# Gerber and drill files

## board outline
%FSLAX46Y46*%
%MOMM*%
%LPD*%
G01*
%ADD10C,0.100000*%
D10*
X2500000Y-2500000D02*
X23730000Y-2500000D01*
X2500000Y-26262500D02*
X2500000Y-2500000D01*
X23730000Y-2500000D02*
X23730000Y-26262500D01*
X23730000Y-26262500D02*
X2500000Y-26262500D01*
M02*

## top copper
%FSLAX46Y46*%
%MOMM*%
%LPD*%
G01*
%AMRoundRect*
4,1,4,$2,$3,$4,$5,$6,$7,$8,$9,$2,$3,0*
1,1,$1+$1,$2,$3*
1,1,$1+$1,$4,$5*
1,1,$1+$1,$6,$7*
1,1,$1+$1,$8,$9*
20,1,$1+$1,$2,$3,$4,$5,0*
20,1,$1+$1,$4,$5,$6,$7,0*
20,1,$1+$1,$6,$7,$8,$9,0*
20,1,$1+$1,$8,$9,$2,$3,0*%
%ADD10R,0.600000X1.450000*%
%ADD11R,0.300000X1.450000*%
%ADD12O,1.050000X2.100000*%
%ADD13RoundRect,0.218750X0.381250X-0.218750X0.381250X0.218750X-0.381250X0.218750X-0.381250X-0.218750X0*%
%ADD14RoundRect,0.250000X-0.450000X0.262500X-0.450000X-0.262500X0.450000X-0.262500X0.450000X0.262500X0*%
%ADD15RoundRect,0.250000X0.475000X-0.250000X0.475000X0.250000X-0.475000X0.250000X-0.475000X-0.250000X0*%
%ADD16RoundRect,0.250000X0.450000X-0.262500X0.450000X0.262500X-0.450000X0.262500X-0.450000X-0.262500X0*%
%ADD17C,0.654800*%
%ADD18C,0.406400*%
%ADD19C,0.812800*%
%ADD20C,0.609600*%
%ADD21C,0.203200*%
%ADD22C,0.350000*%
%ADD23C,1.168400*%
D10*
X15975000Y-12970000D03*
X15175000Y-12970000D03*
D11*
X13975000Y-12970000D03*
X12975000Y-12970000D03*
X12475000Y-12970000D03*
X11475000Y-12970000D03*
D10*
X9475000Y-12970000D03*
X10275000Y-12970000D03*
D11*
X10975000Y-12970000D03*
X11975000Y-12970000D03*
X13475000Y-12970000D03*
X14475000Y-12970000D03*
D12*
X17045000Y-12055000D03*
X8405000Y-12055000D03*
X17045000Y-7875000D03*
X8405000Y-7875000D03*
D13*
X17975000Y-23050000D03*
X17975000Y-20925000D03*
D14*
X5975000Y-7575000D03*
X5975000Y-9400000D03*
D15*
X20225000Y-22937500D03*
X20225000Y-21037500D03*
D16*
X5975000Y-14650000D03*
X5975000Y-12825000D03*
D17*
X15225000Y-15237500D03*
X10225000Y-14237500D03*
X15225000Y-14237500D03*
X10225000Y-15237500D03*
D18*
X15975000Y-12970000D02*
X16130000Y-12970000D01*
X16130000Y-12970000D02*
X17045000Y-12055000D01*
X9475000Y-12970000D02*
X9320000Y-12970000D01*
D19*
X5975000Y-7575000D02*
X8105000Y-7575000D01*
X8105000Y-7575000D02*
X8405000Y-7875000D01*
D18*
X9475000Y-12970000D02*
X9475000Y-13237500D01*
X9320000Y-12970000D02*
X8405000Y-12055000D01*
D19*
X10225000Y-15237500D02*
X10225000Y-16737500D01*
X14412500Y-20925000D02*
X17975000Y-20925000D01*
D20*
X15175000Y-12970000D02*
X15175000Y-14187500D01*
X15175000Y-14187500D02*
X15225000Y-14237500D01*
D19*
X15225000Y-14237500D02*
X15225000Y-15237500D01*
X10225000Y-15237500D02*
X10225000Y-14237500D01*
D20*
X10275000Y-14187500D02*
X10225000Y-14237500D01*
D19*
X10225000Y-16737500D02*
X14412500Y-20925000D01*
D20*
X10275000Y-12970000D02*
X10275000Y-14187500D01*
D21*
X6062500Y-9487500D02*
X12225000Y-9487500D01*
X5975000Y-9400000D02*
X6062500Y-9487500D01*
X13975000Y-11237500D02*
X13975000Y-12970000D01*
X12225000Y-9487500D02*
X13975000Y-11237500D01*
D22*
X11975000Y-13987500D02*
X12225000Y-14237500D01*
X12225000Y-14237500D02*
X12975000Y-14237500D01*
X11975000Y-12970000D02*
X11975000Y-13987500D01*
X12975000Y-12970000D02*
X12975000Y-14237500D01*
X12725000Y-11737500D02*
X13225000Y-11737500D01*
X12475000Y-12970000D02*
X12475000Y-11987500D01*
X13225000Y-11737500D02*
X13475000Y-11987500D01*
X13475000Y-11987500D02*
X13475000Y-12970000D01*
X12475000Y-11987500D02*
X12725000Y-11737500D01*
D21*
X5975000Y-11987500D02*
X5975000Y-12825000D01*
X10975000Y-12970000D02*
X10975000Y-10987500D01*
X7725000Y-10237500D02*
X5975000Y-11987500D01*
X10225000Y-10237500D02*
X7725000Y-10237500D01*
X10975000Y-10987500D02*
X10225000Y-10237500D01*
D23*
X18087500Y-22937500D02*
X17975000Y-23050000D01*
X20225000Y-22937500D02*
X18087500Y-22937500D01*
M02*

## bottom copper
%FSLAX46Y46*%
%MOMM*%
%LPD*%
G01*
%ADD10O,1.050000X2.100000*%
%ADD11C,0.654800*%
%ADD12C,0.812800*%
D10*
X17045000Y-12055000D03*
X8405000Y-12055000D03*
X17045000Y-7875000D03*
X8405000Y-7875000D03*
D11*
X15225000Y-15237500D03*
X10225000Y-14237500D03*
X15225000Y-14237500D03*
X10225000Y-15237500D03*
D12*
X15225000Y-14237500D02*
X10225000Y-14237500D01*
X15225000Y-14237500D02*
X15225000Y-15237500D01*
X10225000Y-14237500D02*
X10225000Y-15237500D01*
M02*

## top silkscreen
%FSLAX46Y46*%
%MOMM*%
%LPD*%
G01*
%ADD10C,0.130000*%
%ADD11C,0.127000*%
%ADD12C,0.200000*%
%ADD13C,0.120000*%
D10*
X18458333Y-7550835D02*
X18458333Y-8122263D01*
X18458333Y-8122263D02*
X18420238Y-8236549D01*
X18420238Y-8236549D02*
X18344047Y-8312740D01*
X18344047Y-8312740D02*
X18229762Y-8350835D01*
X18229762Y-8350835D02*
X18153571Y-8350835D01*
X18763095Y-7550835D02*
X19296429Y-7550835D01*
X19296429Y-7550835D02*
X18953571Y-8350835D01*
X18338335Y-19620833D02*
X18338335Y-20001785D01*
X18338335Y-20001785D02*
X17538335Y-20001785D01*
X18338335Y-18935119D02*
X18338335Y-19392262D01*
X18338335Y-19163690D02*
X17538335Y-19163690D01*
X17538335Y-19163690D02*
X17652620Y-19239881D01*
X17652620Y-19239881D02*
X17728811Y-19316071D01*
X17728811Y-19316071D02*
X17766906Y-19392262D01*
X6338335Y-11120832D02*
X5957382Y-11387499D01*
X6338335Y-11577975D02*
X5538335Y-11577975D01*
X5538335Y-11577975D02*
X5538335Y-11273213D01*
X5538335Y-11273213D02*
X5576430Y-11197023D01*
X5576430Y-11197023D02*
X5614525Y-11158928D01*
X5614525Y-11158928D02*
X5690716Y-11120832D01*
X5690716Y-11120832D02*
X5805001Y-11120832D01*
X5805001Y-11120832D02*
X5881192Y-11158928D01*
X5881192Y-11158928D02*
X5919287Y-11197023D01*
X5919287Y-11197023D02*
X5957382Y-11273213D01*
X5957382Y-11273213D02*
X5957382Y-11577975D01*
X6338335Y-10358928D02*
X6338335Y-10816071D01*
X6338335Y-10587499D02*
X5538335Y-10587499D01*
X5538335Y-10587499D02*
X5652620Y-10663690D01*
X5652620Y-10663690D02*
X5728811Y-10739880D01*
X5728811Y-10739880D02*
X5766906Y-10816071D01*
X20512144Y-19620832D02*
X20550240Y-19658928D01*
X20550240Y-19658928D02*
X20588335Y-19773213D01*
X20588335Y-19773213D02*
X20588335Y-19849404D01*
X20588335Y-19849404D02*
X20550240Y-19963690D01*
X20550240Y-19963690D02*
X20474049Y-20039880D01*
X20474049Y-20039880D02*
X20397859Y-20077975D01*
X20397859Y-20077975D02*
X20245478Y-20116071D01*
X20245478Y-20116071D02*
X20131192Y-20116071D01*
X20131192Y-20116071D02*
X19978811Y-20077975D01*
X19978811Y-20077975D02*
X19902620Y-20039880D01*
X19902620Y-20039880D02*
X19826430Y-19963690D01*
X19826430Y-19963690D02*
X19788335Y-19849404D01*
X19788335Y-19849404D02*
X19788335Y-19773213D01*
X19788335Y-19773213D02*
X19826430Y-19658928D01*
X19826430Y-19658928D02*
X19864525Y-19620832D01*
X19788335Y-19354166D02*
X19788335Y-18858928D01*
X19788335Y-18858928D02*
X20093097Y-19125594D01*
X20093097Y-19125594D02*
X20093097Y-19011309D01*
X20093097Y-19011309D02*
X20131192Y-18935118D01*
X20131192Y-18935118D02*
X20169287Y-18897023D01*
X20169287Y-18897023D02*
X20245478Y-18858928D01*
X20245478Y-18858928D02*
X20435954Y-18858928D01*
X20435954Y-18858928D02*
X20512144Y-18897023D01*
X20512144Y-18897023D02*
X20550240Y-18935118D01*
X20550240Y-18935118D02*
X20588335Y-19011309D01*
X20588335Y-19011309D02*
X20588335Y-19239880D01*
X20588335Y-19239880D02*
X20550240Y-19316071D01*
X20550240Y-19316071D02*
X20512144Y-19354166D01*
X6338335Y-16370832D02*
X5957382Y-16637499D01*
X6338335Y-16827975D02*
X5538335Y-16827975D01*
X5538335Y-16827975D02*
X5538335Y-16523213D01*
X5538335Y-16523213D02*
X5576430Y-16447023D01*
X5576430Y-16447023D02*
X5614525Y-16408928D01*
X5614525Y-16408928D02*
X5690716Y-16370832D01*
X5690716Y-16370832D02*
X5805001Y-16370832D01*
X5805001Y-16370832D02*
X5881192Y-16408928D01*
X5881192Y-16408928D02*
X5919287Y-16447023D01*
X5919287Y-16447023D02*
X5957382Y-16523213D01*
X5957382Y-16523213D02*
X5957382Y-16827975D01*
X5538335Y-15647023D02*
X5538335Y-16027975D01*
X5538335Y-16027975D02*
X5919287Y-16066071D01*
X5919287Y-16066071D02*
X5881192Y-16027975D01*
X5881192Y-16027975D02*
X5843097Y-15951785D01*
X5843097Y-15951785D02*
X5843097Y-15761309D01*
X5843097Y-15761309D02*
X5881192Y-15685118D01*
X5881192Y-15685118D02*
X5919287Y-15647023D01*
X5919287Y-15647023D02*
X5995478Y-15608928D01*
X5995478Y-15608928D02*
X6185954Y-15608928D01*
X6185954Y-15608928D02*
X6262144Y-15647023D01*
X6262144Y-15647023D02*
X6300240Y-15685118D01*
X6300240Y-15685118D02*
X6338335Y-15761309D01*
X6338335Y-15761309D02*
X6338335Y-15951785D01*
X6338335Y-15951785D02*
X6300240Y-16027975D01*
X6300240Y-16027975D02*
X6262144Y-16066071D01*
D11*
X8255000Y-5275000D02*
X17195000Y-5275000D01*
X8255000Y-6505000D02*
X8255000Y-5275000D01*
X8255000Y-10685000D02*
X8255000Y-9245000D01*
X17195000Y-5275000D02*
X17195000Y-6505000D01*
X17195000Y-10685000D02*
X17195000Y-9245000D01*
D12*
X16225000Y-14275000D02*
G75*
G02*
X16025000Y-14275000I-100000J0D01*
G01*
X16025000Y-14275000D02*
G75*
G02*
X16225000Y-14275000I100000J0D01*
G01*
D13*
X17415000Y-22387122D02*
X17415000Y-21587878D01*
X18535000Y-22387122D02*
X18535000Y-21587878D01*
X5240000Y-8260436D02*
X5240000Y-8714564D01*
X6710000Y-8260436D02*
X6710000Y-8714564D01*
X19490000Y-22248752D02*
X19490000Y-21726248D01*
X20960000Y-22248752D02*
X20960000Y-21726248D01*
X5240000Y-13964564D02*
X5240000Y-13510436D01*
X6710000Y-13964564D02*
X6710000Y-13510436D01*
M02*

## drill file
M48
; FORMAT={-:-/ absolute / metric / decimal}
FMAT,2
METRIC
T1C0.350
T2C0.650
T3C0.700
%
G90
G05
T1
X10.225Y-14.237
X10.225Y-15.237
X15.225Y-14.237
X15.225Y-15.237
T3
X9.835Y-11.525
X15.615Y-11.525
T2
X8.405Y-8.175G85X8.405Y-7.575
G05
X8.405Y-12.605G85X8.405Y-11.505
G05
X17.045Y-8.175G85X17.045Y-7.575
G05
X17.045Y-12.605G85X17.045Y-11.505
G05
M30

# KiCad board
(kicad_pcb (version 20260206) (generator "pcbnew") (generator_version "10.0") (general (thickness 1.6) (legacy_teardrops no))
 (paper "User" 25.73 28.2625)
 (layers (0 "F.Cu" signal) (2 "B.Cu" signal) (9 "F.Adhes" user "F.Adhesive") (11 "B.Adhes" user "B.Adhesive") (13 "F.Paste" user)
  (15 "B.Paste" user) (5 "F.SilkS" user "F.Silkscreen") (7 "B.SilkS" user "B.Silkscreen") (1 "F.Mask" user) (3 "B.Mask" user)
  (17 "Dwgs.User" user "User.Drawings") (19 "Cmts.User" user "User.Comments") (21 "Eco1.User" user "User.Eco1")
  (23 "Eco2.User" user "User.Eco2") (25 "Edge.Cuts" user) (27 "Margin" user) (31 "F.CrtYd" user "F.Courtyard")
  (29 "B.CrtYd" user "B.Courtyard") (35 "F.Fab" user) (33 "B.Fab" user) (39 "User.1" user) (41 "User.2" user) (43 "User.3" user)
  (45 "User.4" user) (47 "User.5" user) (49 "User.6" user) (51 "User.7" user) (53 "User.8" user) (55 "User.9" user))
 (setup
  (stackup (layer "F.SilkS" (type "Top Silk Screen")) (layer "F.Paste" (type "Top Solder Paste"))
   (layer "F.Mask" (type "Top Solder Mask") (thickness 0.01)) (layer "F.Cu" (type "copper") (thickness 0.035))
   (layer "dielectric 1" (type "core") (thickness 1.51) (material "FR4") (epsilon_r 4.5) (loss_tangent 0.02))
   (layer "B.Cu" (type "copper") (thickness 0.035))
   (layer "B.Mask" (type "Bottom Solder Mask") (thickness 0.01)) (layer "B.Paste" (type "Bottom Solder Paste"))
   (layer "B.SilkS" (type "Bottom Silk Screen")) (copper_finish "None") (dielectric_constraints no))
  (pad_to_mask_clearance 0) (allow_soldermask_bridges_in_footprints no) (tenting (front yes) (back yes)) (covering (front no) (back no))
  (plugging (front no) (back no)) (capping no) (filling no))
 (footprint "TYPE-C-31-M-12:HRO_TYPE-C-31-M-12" (layer "F.Cu") (at 12.725 7.875 180)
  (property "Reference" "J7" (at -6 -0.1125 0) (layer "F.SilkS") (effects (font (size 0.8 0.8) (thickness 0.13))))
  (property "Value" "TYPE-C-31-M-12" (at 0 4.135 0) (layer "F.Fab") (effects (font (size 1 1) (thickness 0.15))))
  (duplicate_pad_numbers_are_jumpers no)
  (fp_line (start 4.47 2.6) (end -4.47 2.6) (stroke (width 0.127) (type solid)) (layer "F.SilkS"))
  (fp_line (start 4.47 1.37) (end 4.47 2.6) (stroke (width 0.127) (type solid)) (layer "F.SilkS"))
  (fp_line (start 4.47 -2.81) (end 4.47 -1.37) (stroke (width 0.127) (type solid)) (layer "F.SilkS"))
  (fp_line (start -4.47 2.6) (end -4.47 1.37) (stroke (width 0.127) (type solid)) (layer "F.SilkS"))
  (fp_line (start -4.47 -2.81) (end -4.47 -1.37) (stroke (width 0.127) (type solid)) (layer "F.SilkS"))
  (fp_circle (center -3.4 -6.4) (end -3.3 -6.4) (stroke (width 0.2) (type solid)) (fill no) (layer "F.SilkS"))
  (pad "" np_thru_hole circle (at -2.89 -3.65 180) (size 0.7 0.7) (drill 0.7) (layers "*.Cu" "*.Mask"))
  (pad "" np_thru_hole circle (at 2.89 -3.65 180) (size 0.7 0.7) (drill 0.7) (layers "*.Cu" "*.Mask"))
  (pad "A1B12" smd rect (at -3.25 -5.095 180) (size 0.6 1.45) (layers "F.Cu" "F.Mask" "F.Paste") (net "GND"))
  (pad "A4B9" smd rect (at -2.45 -5.095 180) (size 0.6 1.45) (layers "F.Cu" "F.Mask" "F.Paste") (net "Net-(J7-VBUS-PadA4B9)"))
  (pad "A5" smd rect (at -1.25 -5.095 180) (size 0.3 1.45) (layers "F.Cu" "F.Mask" "F.Paste") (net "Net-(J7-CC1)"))
  (pad "A6" smd rect (at -0.25 -5.095 180) (size 0.3 1.45) (layers "F.Cu" "F.Mask" "F.Paste") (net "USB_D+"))
  (pad "A7" smd rect (at 0.25 -5.095 180) (size 0.3 1.45) (layers "F.Cu" "F.Mask" "F.Paste") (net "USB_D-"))
  (pad "A8" smd rect (at 1.25 -5.095 180) (size 0.3 1.45) (layers "F.Cu" "F.Mask" "F.Paste") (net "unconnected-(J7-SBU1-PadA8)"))
  (pad "B1A12" smd rect (at 3.25 -5.095 180) (size 0.6 1.45) (layers "F.Cu" "F.Mask" "F.Paste") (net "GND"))
  (pad "B4A9" smd rect (at 2.45 -5.095 180) (size 0.6 1.45) (layers "F.Cu" "F.Mask" "F.Paste") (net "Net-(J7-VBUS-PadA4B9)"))
  (pad "B5" smd rect (at 1.75 -5.095 180) (size 0.3 1.45) (layers "F.Cu" "F.Mask" "F.Paste") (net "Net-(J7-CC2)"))
  (pad "B6" smd rect (at 0.75 -5.095 180) (size 0.3 1.45) (layers "F.Cu" "F.Mask" "F.Paste") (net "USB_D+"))
  (pad "B7" smd rect (at -0.75 -5.095 180) (size 0.3 1.45) (layers "F.Cu" "F.Mask" "F.Paste") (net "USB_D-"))
  (pad "B8" smd rect (at -1.75 -5.095 180) (size 0.3 1.45) (layers "F.Cu" "F.Mask" "F.Paste") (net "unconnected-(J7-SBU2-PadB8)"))
  (pad "S1" thru_hole oval (at -4.32 -4.18 180) (size 1.05 2.1) (drill oval 0.65 1.75) (layers "*.Cu" "*.Mask") (remove_unused_layers no)
   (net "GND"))
  (pad "S2" thru_hole oval (at 4.32 -4.18 180) (size 1.05 2.1) (drill oval 0.65 1.75) (layers "*.Cu" "*.Mask") (remove_unused_layers no)
   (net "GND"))
  (pad "S3" thru_hole oval (at -4.32 0 180) (size 1.05 2.1) (drill oval 0.65 1.25) (layers "*.Cu" "*.Mask") (remove_unused_layers no)
   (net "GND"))
  (pad "S4" thru_hole oval (at 4.32 0 180) (size 1.05 2.1) (drill oval 0.65 1.25) (layers "*.Cu" "*.Mask") (remove_unused_layers no)
   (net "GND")))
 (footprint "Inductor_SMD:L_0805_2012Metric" (layer "F.Cu") (at 17.975 21.9875 90)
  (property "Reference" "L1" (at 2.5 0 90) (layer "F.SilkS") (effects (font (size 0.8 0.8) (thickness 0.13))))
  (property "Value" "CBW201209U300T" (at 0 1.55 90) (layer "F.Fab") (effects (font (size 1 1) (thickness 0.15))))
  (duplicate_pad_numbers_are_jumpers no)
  (fp_line (start -0.399622 -0.56) (end 0.399622 -0.56) (stroke (width 0.12) (type solid)) (layer "F.SilkS"))
  (fp_line (start -0.399622 0.56) (end 0.399622 0.56) (stroke (width 0.12) (type solid)) (layer "F.SilkS"))
  (pad "1" smd roundrect (at -1.0625 0 90) (size 0.875 1.2) (layers "F.Cu" "F.Mask" "F.Paste") (roundrect_rratio 0.25) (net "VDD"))
  (pad "2" smd roundrect (at 1.0625 0 90) (size 0.875 1.2) (layers "F.Cu" "F.Mask" "F.Paste") (roundrect_rratio 0.25)
   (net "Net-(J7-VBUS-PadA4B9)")))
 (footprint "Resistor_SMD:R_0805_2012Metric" (layer "F.Cu") (at 5.975 8.4875 -90)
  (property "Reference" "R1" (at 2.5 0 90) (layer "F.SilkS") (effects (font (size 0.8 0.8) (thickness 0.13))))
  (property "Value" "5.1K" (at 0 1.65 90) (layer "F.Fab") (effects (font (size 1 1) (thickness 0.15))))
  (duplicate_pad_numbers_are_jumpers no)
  (fp_line (start -0.227064 0.735) (end 0.227064 0.735) (stroke (width 0.12) (type solid)) (layer "F.SilkS"))
  (fp_line (start -0.227064 -0.735) (end 0.227064 -0.735) (stroke (width 0.12) (type solid)) (layer "F.SilkS"))
  (pad "1" smd roundrect (at -0.9125 0 270) (size 1.025 1.4) (layers "F.Cu" "F.Mask" "F.Paste") (roundrect_rratio 0.243902) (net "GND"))
  (pad "2" smd roundrect (at 0.9125 0 270) (size 1.025 1.4) (layers "F.Cu" "F.Mask" "F.Paste") (roundrect_rratio 0.243902)
   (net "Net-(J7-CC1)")))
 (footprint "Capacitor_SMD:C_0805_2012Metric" (layer "F.Cu") (at 20.225 21.9875 90)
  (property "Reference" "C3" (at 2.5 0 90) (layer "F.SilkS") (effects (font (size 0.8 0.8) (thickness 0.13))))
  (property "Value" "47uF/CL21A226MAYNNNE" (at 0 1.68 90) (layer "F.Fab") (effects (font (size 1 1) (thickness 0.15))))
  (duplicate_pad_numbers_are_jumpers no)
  (fp_line (start -0.261252 -0.735) (end 0.261252 -0.735) (stroke (width 0.12) (type solid)) (layer "F.SilkS"))
  (fp_line (start -0.261252 0.735) (end 0.261252 0.735) (stroke (width 0.12) (type solid)) (layer "F.SilkS"))
  (pad "1" smd roundrect (at -0.95 0 90) (size 1 1.45) (layers "F.Cu" "F.Mask" "F.Paste") (roundrect_rratio 0.25) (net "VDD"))
  (pad "2" smd roundrect (at 0.95 0 90) (size 1 1.45) (layers "F.Cu" "F.Mask" "F.Paste") (roundrect_rratio 0.25) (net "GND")))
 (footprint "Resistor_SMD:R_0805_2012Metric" (layer "F.Cu") (at 5.975 13.7375 90)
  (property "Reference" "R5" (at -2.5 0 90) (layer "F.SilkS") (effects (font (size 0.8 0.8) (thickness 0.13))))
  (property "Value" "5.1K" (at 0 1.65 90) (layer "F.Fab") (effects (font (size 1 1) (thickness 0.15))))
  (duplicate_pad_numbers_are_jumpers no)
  (fp_line (start -0.227064 -0.735) (end 0.227064 -0.735) (stroke (width 0.12) (type solid)) (layer "F.SilkS"))
  (fp_line (start -0.227064 0.735) (end 0.227064 0.735) (stroke (width 0.12) (type solid)) (layer "F.SilkS"))
  (pad "1" smd roundrect (at -0.9125 0 90) (size 1.025 1.4) (layers "F.Cu" "F.Mask" "F.Paste") (roundrect_rratio 0.243902) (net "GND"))
  (pad "2" smd roundrect (at 0.9125 0 90) (size 1.025 1.4) (layers "F.Cu" "F.Mask" "F.Paste") (roundrect_rratio 0.243902)
   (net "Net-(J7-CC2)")))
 (gr_line (start 2.5 2.5) (end 23.73 2.5) (stroke (width 0.1) (type default)) (layer "Edge.Cuts"))
 (gr_line (start 2.5 26.2625) (end 2.5 2.5) (stroke (width 0.1) (type default)) (layer "Edge.Cuts"))
 (gr_line (start 23.73 2.5) (end 23.73 26.2625) (stroke (width 0.1) (type default)) (layer "Edge.Cuts"))
 (gr_line (start 23.73 26.2625) (end 2.5 26.2625) (stroke (width 0.1) (type default)) (layer "Edge.Cuts"))
 (segment (start 15.975 12.97) (end 16.13 12.97) (width 0.4064) (layer "F.Cu") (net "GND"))
 (segment (start 16.13 12.97) (end 17.045 12.055) (width 0.4064) (layer "F.Cu") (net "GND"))
 (segment (start 9.475 12.97) (end 9.32 12.97) (width 0.4064) (layer "F.Cu") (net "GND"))
 (segment (start 5.975 7.575) (end 8.105 7.575) (width 0.8128) (layer "F.Cu") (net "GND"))
 (segment (start 8.105 7.575) (end 8.405 7.875) (width 0.8128) (layer "F.Cu") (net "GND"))
 (segment (start 9.475 12.97) (end 9.475 13.2375) (width 0.4064) (layer "F.Cu") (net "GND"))
 (segment (start 9.32 12.97) (end 8.405 12.055) (width 0.4064) (layer "F.Cu") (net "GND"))
 (segment (start 10.225 15.2375) (end 10.225 16.7375) (width 0.8128) (layer "F.Cu") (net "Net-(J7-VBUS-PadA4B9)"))
 (segment (start 14.4125 20.925) (end 17.975 20.925) (width 0.8128) (layer "F.Cu") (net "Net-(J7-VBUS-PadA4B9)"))
 (segment (start 15.175 12.97) (end 15.175 14.1875) (width 0.6096) (layer "F.Cu") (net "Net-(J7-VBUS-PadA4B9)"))
 (segment (start 15.175 14.1875) (end 15.225 14.2375) (width 0.6096) (layer "F.Cu") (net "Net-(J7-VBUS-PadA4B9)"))
 (segment (start 15.225 14.2375) (end 15.225 15.2375) (width 0.8128) (layer "F.Cu") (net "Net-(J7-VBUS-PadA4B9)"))
 (segment (start 10.225 15.2375) (end 10.225 14.2375) (width 0.8128) (layer "F.Cu") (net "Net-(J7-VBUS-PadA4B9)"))
 (segment (start 10.275 14.1875) (end 10.225 14.2375) (width 0.6096) (layer "F.Cu") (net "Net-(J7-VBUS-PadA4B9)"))
 (segment (start 10.225 16.7375) (end 14.4125 20.925) (width 0.8128) (layer "F.Cu") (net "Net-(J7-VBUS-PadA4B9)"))
 (segment (start 10.275 12.97) (end 10.275 14.1875) (width 0.6096) (layer "F.Cu") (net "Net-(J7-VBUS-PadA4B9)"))
 (via (at 15.225 15.2375) (size 0.6548) (drill 0.35) (layers "F.Cu" "B.Cu") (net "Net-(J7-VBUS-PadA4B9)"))
 (via (at 10.225 14.2375) (size 0.6548) (drill 0.35) (layers "F.Cu" "B.Cu") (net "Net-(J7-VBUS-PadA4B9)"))
 (via (at 15.225 14.2375) (size 0.6548) (drill 0.35) (layers "F.Cu" "B.Cu") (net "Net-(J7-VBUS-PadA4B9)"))
 (via (at 10.225 15.2375) (size 0.6548) (drill 0.35) (layers "F.Cu" "B.Cu") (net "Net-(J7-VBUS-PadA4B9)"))
 (segment (start 15.225 14.2375) (end 10.225 14.2375) (width 0.8128) (layer "B.Cu") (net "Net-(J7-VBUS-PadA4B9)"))
 (segment (start 15.225 14.2375) (end 15.225 15.2375) (width 0.8128) (layer "B.Cu") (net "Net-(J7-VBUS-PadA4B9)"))
 (segment (start 10.225 14.2375) (end 10.225 15.2375) (width 0.8128) (layer "B.Cu") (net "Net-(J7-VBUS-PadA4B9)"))
 (segment (start 6.0625 9.4875) (end 12.225 9.4875) (width 0.2032) (layer "F.Cu") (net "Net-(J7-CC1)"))
 (segment (start 5.975 9.4) (end 6.0625 9.4875) (width 0.2032) (layer "F.Cu") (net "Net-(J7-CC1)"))
 (segment (start 13.975 11.2375) (end 13.975 12.97) (width 0.2032) (layer "F.Cu") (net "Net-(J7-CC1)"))
 (segment (start 12.225 9.4875) (end 13.975 11.2375) (width 0.2032) (layer "F.Cu") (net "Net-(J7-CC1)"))
 (segment (start 11.975 13.9875) (end 12.225 14.2375) (width 0.35) (layer "F.Cu") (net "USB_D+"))
 (segment (start 12.225 14.2375) (end 12.975 14.2375) (width 0.35) (layer "F.Cu") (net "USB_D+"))
 (segment (start 11.975 12.97) (end 11.975 13.9875) (width 0.35) (layer "F.Cu") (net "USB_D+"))
 (segment (start 12.975 12.97) (end 12.975 14.2375) (width 0.35) (layer "F.Cu") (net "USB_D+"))
 (segment (start 12.725 11.7375) (end 13.225 11.7375) (width 0.35) (layer "F.Cu") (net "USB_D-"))
 (segment (start 12.475 12.97) (end 12.475 11.9875) (width 0.35) (layer "F.Cu") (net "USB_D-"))
 (segment (start 13.225 11.7375) (end 13.475 11.9875) (width 0.35) (layer "F.Cu") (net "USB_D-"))
 (segment (start 13.475 11.9875) (end 13.475 12.97) (width 0.35) (layer "F.Cu") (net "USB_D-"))
 (segment (start 12.475 11.9875) (end 12.725 11.7375) (width 0.35) (layer "F.Cu") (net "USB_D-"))
 (segment (start 5.975 11.9875) (end 5.975 12.825) (width 0.2032) (layer "F.Cu") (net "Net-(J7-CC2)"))
 (segment (start 10.975 12.97) (end 10.975 10.9875) (width 0.2032) (layer "F.Cu") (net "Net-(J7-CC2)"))
 (segment (start 7.725 10.2375) (end 5.975 11.9875) (width 0.2032) (layer "F.Cu") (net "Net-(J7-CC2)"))
 (segment (start 10.225 10.2375) (end 7.725 10.2375) (width 0.2032) (layer "F.Cu") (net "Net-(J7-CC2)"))
 (segment (start 10.975 10.9875) (end 10.225 10.2375) (width 0.2032) (layer "F.Cu") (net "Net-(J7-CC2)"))
 (segment (start 18.0875 22.9375) (end 17.975 23.05) (width 1.1684) (layer "F.Cu") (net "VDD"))
 (segment (start 20.225 22.9375) (end 18.0875 22.9375) (width 1.1684) (layer "F.Cu") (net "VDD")))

